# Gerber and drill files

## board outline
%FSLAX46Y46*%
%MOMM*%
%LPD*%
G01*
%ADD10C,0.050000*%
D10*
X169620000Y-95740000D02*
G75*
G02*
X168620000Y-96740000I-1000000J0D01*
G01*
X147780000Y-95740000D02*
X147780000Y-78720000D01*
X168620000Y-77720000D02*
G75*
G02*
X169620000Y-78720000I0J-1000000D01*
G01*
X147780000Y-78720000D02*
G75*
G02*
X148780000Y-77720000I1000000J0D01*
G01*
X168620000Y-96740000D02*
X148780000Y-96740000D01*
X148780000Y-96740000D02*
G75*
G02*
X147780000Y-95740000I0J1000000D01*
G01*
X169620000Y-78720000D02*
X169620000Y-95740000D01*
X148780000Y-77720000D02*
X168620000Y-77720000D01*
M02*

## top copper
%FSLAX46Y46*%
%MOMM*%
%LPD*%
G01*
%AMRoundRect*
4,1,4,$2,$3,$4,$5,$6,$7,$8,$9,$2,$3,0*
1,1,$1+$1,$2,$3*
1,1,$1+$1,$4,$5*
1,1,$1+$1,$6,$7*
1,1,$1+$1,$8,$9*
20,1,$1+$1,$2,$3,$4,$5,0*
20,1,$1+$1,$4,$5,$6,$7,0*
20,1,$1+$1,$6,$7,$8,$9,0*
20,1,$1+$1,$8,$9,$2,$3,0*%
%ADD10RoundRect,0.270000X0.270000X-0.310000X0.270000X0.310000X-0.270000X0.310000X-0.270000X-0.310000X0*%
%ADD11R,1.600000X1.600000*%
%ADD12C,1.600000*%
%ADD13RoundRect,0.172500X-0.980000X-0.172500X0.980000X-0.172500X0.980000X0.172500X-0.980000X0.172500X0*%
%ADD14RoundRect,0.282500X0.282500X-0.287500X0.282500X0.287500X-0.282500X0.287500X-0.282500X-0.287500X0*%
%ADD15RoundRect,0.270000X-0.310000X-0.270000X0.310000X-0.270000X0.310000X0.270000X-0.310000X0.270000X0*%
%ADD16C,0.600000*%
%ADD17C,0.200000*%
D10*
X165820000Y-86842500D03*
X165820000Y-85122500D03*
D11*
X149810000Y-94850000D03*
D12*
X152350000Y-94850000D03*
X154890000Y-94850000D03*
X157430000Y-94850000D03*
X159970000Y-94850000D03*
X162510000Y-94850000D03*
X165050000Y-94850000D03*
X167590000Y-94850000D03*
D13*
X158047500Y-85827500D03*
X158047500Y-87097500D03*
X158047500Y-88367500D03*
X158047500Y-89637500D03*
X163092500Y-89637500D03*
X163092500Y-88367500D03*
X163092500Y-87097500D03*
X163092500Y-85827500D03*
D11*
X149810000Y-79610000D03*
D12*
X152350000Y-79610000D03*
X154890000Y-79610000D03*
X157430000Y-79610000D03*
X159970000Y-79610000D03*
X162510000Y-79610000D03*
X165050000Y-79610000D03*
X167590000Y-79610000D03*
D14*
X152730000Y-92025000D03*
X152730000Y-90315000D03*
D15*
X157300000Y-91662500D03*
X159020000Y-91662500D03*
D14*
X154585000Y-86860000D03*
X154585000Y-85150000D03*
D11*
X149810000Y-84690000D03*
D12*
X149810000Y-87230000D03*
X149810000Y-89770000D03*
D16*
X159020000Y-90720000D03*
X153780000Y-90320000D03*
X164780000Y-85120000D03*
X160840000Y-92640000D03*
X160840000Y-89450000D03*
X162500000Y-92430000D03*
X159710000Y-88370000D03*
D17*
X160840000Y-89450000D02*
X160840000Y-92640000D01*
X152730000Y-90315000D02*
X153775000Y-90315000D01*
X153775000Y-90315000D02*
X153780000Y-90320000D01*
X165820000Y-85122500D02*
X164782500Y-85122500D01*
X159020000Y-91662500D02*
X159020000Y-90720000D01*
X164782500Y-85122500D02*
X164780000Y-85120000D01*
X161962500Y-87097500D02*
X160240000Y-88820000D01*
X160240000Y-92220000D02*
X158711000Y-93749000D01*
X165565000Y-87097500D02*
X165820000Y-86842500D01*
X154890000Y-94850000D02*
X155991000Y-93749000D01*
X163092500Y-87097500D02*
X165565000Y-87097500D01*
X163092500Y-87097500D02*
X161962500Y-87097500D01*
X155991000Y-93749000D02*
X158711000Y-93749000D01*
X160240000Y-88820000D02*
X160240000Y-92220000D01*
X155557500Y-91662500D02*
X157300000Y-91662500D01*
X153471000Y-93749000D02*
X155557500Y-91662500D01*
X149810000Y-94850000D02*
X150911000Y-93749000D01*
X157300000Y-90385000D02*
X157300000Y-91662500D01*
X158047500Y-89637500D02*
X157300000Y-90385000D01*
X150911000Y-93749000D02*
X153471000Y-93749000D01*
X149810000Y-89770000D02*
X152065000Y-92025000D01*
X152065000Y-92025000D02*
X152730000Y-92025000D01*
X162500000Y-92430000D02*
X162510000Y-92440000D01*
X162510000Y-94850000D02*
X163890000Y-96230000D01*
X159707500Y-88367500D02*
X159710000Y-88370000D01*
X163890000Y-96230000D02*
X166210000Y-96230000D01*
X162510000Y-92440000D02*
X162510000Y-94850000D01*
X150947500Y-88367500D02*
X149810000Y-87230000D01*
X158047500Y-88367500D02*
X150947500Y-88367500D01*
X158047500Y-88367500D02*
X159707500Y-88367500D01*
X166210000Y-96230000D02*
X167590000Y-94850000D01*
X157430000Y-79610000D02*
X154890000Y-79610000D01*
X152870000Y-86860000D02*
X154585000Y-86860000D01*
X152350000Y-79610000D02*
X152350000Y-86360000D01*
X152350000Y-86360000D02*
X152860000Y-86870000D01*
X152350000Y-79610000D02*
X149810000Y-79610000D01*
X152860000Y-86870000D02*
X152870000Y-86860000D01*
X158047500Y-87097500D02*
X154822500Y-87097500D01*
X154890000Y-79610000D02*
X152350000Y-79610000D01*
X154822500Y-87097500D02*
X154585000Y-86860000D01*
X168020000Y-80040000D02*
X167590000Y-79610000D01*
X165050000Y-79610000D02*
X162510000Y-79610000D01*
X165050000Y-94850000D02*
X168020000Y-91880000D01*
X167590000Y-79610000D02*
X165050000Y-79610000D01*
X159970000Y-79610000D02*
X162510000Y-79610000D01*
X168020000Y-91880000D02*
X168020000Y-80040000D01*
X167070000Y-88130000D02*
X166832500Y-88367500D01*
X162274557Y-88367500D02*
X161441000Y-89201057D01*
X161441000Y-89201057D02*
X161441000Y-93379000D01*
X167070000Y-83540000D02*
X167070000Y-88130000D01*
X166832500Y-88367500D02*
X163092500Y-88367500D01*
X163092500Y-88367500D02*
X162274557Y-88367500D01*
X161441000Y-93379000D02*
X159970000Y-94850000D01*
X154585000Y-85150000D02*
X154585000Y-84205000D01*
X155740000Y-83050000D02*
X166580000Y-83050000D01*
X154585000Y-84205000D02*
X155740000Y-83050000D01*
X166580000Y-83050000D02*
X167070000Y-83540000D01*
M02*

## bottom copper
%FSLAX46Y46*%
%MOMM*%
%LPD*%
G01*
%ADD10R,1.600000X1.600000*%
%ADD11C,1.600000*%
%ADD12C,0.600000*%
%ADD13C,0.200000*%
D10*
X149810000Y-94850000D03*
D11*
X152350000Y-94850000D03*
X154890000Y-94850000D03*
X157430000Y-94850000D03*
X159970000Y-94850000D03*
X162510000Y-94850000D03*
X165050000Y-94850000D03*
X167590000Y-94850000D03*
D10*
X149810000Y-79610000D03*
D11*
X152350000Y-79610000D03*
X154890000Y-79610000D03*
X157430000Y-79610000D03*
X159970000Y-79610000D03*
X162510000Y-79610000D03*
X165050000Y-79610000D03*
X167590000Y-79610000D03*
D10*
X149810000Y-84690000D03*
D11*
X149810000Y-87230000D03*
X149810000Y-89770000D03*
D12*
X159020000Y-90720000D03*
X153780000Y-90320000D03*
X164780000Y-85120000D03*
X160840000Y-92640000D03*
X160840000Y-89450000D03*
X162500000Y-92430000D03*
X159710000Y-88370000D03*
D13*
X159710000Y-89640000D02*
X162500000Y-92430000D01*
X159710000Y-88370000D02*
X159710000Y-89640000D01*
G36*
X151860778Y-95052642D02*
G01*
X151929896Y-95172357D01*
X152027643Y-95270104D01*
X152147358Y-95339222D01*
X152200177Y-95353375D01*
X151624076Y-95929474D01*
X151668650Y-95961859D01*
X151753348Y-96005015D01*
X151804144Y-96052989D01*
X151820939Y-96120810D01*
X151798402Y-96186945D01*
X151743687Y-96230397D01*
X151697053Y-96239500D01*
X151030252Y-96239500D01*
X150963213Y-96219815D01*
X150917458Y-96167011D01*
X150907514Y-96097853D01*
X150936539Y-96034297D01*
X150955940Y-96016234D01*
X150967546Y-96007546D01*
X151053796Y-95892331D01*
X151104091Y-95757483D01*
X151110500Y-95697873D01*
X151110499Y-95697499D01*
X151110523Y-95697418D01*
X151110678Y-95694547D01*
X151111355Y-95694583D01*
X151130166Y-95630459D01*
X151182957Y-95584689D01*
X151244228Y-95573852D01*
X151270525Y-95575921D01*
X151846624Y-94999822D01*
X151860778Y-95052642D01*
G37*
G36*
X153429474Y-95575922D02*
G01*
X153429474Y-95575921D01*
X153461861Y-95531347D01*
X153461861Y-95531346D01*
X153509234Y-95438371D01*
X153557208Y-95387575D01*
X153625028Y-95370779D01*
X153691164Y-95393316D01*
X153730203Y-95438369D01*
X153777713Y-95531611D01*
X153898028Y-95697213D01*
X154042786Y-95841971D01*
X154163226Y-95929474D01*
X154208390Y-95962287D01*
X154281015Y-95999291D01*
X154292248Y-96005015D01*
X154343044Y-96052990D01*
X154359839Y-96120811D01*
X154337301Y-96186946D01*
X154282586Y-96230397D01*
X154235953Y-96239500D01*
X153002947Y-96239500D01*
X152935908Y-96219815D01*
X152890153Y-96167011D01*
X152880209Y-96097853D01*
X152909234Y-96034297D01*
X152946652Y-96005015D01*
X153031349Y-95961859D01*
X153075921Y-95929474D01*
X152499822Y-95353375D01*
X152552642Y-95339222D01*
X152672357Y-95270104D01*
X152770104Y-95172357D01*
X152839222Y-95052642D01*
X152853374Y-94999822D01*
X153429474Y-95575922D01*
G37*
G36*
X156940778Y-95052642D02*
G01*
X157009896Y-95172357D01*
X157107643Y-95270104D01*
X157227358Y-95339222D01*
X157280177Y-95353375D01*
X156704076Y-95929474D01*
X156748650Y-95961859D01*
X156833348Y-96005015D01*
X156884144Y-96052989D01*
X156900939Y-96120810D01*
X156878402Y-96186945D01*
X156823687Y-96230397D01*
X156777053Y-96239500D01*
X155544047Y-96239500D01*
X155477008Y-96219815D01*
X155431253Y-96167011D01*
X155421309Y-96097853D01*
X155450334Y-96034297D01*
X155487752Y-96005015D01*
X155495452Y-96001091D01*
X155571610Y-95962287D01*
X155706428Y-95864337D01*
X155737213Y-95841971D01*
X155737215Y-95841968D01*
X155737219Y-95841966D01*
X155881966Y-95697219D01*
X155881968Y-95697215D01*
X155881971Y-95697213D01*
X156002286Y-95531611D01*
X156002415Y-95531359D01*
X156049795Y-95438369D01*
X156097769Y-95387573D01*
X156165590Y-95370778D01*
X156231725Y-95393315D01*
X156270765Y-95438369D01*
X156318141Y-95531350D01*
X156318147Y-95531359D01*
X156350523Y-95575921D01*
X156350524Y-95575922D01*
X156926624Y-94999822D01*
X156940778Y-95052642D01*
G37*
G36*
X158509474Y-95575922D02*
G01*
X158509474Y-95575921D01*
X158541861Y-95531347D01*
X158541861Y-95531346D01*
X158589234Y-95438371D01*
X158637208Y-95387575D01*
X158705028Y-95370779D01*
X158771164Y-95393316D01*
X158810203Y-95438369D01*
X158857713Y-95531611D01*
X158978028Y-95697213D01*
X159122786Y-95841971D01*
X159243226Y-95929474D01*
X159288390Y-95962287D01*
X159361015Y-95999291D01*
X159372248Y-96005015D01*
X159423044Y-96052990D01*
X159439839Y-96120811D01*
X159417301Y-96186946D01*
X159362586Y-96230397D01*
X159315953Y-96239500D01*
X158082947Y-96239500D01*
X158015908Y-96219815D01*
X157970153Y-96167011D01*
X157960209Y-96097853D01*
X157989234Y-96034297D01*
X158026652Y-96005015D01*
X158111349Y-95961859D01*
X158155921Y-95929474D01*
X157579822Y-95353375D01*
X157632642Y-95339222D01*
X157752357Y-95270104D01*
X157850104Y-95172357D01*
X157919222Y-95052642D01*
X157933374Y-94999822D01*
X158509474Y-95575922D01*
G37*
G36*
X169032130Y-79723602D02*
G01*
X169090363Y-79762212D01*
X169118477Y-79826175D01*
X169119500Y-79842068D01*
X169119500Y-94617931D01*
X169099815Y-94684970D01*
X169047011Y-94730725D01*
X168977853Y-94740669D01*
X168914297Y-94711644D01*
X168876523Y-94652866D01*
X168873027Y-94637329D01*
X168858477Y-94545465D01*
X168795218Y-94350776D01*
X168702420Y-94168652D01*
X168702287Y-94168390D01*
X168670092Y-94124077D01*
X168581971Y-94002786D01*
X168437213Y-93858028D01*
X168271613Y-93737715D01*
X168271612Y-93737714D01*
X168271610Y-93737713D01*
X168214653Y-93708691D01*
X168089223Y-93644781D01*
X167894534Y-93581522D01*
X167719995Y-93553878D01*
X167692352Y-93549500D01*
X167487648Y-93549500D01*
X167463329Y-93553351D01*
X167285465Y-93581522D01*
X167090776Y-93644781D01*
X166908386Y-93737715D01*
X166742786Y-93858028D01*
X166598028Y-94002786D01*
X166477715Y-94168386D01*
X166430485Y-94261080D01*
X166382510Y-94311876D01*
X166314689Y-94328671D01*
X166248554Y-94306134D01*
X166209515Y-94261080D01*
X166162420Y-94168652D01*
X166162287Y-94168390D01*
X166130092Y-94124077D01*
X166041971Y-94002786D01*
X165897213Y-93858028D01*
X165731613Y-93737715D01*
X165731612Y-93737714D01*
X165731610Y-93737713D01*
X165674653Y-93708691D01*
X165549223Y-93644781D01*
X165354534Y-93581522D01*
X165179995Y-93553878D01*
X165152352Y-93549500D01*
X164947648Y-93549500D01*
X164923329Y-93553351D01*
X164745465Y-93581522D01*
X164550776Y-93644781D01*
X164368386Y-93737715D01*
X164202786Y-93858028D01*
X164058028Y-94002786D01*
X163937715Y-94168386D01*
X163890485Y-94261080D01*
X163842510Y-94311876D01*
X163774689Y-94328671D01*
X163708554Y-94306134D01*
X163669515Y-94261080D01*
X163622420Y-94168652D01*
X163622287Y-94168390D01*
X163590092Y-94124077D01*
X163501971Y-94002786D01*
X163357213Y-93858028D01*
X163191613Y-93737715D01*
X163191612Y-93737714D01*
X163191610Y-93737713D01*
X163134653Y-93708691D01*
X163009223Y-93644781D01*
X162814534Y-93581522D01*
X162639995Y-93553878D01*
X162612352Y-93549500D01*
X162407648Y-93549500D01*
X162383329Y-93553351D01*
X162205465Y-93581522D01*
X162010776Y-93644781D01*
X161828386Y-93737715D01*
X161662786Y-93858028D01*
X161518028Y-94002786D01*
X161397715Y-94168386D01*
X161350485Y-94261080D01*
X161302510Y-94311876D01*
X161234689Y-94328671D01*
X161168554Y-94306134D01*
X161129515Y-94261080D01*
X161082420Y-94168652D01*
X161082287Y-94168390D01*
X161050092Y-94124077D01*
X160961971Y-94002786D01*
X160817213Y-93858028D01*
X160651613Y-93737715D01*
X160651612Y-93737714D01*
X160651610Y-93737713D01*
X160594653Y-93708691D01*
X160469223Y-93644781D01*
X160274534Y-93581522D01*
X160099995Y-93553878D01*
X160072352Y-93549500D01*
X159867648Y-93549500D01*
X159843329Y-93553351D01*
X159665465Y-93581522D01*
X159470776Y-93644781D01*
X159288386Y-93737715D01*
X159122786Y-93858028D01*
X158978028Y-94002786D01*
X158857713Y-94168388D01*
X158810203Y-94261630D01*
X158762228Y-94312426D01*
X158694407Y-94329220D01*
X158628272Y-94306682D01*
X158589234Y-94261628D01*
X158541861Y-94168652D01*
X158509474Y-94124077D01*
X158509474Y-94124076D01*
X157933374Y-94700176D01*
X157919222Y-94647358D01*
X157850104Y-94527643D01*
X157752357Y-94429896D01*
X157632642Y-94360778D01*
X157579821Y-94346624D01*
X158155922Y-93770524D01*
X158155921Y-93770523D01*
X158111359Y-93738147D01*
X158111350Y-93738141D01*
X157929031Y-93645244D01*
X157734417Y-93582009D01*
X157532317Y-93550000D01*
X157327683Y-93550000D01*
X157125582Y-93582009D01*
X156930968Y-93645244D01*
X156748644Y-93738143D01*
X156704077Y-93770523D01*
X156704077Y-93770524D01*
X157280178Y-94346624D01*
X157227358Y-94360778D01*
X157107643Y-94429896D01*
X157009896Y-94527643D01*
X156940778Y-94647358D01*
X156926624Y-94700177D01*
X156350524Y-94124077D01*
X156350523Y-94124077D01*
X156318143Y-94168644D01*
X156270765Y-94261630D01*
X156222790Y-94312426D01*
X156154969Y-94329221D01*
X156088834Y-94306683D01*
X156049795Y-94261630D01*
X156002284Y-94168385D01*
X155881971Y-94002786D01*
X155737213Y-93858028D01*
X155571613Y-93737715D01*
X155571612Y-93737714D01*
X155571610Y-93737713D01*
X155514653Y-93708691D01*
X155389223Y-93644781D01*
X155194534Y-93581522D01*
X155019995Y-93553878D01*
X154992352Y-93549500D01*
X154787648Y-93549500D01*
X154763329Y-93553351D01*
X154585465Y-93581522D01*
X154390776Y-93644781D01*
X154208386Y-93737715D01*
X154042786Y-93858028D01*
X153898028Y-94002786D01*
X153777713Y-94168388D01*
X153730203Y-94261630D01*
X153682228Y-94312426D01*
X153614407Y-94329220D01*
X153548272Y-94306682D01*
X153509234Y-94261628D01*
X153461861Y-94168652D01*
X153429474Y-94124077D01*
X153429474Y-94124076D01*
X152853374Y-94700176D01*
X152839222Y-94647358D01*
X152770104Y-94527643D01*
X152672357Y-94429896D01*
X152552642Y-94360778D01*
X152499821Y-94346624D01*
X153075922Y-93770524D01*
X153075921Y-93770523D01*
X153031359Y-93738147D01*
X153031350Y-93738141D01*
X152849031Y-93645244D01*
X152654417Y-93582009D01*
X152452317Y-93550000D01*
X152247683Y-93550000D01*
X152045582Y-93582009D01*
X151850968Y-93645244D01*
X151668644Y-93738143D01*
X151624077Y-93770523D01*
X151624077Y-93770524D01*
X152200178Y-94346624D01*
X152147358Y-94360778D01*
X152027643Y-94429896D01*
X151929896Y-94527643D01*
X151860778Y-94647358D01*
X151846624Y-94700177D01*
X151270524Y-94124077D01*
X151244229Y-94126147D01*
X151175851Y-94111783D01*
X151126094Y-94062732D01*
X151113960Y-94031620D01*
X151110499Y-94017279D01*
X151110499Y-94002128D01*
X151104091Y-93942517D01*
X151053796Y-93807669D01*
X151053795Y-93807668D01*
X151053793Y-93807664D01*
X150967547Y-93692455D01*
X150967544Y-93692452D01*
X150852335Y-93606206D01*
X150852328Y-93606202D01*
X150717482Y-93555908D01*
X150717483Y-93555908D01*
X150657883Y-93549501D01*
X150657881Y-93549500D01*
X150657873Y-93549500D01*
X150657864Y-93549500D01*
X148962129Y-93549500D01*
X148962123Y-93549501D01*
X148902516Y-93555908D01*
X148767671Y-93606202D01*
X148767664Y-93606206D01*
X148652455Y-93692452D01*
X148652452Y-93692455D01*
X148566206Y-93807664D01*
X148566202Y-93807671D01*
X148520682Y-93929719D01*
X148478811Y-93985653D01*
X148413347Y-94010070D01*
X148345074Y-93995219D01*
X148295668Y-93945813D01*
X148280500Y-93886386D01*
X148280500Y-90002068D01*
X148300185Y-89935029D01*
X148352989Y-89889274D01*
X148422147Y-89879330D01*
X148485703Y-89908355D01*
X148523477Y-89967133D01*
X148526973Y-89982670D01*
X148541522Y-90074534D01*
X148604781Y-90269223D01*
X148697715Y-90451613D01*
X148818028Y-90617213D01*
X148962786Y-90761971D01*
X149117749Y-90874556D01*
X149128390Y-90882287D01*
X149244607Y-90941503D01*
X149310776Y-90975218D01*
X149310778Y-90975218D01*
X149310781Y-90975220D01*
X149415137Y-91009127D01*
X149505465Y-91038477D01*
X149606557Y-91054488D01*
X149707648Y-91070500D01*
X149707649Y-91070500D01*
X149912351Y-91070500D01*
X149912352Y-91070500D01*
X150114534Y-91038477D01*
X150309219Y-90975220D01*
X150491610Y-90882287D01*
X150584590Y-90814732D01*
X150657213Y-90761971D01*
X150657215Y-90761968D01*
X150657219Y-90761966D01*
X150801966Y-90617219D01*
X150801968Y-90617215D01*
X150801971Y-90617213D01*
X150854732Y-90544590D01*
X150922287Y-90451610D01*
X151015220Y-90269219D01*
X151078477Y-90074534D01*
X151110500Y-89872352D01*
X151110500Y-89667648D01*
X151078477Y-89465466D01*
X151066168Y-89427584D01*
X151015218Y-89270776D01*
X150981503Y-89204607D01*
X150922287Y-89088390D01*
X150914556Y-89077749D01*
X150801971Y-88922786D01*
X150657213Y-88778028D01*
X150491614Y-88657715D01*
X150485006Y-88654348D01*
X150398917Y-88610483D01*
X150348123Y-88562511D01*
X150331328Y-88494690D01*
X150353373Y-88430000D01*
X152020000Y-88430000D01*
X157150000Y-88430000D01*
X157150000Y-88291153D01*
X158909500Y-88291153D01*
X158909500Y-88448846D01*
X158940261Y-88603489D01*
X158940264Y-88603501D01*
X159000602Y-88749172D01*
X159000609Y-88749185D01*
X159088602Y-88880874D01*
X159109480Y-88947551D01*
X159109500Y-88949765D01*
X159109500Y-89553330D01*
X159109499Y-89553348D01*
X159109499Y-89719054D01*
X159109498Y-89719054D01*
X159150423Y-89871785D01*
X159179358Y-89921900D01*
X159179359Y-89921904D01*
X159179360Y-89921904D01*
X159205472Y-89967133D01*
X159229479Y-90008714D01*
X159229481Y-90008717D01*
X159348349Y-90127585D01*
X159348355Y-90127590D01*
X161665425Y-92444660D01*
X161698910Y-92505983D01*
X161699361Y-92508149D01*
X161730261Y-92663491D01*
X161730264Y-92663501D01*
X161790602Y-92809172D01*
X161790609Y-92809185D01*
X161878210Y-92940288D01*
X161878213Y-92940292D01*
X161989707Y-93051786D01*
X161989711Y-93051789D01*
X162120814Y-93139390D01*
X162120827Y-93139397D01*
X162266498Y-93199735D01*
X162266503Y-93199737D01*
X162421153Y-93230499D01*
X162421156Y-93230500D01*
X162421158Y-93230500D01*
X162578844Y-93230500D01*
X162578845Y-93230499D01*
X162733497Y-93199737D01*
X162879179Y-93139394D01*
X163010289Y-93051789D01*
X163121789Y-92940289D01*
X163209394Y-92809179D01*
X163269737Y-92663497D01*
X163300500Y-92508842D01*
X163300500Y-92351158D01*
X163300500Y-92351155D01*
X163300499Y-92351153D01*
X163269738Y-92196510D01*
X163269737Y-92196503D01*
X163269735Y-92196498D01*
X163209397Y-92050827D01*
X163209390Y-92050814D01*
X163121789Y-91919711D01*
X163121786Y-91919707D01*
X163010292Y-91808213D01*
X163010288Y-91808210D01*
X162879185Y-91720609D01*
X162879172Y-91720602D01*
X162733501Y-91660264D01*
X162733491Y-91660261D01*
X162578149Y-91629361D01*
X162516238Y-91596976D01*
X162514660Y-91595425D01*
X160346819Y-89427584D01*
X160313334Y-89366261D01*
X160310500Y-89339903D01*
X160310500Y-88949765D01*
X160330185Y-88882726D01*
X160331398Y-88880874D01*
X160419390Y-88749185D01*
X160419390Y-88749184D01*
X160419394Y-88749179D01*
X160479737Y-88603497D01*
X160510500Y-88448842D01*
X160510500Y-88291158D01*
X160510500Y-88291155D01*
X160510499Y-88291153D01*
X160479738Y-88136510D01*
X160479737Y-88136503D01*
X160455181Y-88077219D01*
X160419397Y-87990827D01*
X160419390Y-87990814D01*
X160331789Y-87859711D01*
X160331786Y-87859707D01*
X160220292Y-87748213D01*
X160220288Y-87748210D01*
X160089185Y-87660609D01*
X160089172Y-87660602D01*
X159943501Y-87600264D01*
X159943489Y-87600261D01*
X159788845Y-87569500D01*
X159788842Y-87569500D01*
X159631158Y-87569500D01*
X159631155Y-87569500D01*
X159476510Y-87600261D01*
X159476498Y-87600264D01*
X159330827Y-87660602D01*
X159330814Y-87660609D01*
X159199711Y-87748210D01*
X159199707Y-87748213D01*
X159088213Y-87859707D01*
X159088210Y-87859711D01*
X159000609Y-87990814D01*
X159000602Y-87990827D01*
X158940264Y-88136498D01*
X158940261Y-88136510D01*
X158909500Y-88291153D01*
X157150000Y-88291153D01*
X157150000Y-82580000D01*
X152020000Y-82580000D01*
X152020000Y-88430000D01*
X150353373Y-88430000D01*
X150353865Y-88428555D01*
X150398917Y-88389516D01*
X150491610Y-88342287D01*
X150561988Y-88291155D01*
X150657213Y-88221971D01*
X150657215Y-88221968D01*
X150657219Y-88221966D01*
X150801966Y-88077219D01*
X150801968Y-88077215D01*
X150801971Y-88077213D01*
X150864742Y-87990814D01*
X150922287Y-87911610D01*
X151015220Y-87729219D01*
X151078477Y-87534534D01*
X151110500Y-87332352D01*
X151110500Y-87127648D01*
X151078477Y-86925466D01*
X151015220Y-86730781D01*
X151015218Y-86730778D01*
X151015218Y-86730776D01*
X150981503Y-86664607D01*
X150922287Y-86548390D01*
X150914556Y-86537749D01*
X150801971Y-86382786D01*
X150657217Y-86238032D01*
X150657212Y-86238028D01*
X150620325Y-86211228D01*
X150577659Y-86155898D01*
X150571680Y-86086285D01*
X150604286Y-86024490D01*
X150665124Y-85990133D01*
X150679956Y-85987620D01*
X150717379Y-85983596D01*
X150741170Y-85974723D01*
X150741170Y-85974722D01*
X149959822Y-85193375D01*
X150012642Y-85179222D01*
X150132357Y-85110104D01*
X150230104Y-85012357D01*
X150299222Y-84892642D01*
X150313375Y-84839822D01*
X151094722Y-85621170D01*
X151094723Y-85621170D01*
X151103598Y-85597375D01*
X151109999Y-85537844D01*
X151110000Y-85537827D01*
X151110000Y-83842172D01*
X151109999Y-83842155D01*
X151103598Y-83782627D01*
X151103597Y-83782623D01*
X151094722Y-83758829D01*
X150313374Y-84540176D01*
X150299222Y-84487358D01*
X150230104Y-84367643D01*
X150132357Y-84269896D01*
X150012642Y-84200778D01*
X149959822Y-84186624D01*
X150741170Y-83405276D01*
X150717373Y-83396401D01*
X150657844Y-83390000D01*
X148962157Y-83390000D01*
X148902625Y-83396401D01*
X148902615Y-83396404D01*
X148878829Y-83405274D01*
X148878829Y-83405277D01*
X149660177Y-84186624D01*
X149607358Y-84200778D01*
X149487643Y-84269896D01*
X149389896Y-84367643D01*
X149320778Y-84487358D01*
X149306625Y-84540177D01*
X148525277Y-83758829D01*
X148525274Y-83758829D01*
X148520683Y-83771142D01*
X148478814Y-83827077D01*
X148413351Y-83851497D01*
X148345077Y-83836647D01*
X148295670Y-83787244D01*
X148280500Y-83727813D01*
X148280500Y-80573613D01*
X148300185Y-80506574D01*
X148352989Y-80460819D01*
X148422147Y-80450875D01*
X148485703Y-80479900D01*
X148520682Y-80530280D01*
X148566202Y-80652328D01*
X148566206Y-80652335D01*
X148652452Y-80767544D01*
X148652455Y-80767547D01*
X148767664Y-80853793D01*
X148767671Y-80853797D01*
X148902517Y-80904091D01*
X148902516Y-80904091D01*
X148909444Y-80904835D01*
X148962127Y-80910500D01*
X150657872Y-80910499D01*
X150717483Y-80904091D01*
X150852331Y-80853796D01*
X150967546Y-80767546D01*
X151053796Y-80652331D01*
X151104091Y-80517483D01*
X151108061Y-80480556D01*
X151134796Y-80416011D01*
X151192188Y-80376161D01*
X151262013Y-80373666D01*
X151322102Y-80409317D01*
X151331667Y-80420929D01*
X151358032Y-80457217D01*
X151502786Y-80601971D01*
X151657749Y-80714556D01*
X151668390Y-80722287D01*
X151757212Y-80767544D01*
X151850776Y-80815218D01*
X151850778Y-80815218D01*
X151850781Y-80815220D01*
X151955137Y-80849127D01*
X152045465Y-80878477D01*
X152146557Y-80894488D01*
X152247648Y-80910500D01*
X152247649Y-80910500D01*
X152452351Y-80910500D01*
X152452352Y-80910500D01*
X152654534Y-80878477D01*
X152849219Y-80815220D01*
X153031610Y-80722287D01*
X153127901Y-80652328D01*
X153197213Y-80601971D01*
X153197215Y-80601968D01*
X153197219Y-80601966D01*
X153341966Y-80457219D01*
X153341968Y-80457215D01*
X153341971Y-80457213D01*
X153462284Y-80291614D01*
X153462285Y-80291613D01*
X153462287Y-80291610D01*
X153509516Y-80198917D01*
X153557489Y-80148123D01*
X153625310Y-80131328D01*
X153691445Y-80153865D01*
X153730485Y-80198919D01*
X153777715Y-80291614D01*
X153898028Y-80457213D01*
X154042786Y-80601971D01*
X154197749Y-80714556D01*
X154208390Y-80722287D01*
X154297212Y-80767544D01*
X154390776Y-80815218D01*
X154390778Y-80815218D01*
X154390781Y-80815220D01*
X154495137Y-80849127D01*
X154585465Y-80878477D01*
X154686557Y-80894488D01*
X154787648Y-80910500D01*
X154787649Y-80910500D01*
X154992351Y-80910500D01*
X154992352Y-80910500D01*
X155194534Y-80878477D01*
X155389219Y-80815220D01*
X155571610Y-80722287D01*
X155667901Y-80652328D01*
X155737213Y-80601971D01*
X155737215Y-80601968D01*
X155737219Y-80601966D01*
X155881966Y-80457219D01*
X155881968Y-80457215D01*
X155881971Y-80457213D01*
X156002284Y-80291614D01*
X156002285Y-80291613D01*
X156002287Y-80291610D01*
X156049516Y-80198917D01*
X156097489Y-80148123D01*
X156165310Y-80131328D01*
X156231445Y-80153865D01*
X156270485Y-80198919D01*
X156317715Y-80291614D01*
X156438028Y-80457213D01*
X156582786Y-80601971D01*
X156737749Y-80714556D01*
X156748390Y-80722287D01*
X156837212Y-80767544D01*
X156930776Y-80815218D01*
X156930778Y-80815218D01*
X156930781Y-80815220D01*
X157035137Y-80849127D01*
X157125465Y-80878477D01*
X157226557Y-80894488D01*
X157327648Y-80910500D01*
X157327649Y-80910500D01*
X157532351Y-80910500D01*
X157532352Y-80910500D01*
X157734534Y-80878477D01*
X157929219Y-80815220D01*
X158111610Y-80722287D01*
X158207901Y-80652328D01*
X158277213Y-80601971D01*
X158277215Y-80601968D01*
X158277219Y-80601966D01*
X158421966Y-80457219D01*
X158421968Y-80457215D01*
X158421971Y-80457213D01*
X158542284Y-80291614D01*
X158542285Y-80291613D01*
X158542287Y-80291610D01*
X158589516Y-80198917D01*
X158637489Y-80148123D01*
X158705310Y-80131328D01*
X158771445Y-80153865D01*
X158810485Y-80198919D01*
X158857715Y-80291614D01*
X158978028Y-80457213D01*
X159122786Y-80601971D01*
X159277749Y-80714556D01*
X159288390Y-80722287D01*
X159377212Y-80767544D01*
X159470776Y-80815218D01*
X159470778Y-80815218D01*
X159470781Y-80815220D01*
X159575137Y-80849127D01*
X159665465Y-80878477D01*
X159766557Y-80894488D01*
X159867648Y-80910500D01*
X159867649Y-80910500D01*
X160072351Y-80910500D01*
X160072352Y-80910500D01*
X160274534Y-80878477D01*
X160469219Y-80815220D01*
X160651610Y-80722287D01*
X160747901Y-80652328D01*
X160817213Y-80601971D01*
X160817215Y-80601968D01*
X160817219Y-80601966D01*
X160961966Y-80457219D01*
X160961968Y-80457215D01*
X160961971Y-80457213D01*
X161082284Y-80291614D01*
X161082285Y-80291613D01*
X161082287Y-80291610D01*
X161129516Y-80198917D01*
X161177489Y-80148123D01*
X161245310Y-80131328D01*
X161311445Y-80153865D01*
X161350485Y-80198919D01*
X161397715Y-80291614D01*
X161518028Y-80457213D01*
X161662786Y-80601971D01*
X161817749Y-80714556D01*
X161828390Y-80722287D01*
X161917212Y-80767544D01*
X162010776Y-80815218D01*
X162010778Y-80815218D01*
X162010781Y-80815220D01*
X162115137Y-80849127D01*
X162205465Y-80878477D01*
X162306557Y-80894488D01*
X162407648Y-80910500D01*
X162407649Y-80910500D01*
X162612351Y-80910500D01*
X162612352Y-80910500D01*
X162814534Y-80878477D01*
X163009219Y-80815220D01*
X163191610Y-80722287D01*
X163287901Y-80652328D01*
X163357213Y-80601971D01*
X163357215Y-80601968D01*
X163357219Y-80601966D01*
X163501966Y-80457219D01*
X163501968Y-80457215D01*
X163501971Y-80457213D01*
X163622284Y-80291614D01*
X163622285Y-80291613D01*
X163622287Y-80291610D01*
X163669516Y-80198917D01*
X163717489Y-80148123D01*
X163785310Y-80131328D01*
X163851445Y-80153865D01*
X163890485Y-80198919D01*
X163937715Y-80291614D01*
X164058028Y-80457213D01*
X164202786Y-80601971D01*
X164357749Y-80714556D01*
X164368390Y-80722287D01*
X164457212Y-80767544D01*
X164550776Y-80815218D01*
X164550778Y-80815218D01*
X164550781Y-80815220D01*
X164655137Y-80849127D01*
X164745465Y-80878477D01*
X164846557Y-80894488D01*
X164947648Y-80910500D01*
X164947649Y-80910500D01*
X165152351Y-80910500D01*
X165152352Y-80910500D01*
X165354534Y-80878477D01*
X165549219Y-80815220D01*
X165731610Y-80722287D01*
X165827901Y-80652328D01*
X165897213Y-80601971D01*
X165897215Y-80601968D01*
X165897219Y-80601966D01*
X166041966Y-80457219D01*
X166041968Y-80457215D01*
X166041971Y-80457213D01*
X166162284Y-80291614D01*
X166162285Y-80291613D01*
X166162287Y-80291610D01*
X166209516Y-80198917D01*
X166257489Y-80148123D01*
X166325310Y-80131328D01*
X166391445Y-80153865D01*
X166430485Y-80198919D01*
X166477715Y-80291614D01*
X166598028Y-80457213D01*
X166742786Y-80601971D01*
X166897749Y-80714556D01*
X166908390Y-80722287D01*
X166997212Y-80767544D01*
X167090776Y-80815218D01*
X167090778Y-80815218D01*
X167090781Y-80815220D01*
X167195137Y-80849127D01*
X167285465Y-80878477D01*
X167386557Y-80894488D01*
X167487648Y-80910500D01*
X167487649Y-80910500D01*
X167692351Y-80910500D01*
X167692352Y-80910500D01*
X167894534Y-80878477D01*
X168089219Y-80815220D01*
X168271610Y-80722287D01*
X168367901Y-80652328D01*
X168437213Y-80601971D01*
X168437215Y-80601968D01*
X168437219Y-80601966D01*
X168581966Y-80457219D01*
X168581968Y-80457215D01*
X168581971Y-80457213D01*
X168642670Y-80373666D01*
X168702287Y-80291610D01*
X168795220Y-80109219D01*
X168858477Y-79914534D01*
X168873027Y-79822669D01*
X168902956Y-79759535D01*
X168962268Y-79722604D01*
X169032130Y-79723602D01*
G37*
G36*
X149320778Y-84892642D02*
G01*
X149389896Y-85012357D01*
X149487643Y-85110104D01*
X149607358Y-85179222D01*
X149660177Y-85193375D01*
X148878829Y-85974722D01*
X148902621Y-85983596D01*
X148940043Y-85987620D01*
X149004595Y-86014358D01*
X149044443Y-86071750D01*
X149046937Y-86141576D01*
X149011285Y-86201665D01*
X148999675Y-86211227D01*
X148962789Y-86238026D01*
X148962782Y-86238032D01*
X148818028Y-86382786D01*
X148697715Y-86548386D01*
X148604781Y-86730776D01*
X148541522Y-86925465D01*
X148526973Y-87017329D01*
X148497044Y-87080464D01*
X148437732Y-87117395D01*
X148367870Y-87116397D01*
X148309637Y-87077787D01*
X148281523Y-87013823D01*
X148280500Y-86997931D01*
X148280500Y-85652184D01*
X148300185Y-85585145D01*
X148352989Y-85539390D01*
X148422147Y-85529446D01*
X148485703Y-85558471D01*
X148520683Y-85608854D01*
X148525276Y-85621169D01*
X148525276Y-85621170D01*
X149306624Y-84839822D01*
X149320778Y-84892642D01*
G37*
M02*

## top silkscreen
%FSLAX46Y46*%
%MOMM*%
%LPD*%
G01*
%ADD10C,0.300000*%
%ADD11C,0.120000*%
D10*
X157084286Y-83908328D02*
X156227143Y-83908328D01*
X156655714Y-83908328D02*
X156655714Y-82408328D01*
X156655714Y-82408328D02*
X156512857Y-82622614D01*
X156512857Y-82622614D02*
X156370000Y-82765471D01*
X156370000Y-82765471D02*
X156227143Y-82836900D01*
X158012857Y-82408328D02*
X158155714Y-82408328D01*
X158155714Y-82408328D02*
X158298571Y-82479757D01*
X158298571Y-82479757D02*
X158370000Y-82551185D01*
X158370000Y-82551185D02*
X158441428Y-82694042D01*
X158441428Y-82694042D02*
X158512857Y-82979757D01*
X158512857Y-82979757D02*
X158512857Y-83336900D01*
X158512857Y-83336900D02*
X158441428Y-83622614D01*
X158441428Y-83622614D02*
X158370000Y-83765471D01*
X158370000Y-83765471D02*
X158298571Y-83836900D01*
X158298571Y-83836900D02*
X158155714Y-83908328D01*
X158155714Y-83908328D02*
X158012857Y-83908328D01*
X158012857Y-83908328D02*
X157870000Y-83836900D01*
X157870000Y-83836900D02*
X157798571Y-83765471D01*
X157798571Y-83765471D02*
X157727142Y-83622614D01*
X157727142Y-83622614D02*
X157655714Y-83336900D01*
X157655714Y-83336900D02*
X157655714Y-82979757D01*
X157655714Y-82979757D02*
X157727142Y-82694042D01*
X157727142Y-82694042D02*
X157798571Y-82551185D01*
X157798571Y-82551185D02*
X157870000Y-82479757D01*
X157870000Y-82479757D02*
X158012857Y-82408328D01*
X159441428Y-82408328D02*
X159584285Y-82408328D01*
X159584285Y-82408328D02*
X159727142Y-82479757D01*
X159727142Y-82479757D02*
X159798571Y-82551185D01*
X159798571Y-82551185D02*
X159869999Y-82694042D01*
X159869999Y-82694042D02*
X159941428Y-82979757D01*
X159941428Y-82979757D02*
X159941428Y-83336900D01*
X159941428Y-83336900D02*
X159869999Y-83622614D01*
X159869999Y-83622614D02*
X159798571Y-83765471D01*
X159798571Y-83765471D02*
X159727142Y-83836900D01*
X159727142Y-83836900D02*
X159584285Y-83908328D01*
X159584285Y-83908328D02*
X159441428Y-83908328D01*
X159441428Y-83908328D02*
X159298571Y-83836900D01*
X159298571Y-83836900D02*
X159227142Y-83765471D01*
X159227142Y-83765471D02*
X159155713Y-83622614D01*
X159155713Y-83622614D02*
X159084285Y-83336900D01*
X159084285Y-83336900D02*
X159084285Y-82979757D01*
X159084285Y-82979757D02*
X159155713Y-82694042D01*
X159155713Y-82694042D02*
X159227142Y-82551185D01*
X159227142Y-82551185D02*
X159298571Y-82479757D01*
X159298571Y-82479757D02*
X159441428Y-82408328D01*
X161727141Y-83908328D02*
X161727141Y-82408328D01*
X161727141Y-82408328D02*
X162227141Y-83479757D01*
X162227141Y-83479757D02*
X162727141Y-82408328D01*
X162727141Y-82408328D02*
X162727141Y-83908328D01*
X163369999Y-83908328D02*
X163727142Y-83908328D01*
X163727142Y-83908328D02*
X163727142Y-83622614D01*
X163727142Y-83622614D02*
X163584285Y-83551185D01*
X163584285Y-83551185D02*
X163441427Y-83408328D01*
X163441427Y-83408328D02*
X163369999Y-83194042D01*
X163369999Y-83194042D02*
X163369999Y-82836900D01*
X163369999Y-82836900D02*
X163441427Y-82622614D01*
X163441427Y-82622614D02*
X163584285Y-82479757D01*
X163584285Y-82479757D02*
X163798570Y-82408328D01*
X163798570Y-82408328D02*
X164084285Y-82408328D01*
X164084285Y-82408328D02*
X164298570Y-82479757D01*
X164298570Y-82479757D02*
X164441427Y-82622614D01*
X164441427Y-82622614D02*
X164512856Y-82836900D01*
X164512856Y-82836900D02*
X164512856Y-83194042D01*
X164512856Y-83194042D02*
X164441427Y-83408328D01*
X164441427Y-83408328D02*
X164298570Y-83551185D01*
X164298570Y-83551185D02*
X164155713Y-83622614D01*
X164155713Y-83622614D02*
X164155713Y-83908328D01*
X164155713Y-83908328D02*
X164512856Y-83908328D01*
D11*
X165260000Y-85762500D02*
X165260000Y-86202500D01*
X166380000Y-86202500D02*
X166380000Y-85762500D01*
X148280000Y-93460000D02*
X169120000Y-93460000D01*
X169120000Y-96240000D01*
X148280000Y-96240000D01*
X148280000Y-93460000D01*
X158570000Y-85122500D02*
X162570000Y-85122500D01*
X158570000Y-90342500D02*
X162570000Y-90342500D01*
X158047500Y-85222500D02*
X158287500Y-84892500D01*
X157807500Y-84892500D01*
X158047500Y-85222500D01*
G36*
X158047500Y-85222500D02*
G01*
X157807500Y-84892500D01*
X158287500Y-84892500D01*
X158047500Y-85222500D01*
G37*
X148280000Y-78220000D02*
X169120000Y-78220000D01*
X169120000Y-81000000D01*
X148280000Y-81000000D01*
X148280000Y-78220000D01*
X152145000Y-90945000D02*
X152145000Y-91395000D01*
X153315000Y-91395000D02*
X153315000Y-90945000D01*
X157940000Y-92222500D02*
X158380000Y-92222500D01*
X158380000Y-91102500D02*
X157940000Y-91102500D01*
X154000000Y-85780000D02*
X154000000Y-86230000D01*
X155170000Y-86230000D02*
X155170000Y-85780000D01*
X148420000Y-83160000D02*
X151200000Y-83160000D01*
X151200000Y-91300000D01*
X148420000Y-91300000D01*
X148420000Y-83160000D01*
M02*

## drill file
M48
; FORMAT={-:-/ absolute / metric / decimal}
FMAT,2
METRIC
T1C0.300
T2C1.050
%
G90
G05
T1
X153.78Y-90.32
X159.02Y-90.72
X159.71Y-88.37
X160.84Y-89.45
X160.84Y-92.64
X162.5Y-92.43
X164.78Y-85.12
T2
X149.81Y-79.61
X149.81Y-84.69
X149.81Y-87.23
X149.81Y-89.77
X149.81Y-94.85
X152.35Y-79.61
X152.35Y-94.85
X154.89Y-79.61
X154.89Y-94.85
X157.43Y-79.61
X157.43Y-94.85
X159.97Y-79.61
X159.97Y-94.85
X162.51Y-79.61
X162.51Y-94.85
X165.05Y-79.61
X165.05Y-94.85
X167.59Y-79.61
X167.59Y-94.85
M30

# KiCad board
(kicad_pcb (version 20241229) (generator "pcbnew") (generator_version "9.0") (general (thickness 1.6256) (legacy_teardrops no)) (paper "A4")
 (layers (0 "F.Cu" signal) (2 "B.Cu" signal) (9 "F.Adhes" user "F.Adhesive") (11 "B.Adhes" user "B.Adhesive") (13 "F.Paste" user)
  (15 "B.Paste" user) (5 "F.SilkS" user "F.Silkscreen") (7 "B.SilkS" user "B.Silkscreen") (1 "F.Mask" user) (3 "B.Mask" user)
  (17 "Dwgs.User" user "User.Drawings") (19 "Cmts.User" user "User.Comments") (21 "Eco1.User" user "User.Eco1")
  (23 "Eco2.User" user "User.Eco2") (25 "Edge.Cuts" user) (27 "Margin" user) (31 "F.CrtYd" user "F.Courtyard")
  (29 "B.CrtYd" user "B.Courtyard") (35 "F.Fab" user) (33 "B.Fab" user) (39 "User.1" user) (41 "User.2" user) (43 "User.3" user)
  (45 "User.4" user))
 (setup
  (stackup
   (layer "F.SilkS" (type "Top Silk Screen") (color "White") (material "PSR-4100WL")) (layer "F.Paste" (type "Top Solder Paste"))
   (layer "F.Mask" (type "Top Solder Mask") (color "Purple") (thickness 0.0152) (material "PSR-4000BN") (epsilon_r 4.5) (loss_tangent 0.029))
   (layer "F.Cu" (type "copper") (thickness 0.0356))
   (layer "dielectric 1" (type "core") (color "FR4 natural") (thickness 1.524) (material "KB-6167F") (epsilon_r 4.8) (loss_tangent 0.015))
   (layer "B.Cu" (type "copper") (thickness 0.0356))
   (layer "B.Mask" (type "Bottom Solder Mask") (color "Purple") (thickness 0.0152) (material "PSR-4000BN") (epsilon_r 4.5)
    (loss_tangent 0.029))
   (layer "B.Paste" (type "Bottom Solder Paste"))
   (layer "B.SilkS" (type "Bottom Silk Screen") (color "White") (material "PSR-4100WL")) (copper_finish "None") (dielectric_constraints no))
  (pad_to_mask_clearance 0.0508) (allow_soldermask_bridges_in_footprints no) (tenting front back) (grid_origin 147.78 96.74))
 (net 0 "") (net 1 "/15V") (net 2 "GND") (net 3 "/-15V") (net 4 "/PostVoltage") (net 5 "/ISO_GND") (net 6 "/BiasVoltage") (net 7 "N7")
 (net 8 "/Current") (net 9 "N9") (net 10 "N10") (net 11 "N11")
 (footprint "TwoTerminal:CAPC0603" (layer "F.Cu") (at 165.82 85.9825 90)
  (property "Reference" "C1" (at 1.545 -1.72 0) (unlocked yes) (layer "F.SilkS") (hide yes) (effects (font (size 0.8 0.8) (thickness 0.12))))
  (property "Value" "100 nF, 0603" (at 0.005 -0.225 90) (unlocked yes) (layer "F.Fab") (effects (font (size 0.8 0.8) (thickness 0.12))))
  (fp_line (start 0.22 -0.56) (end -0.22 -0.56) (stroke (width 0.12) (type default)) (layer "F.SilkS"))
  (fp_line (start -0.22 0.56) (end 0.22 0.56) (stroke (width 0.12) (type default)) (layer "F.SilkS"))
  (pad "1" smd roundrect (at -0.86 0 90) (size 1.16 1.08) (layers "F.Cu" "F.Mask" "F.Paste") (roundrect_rratio 0.25) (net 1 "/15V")
   (thermal_bridge_angle 45))
  (pad "2" smd roundrect (at 0.86 0 90) (size 1.16 1.08) (layers "F.Cu" "F.Mask" "F.Paste") (roundrect_rratio 0.25) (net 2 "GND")
   (thermal_bridge_angle 45)))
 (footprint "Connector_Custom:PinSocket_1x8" (layer "F.Cu") (at 158.7 94.85 90)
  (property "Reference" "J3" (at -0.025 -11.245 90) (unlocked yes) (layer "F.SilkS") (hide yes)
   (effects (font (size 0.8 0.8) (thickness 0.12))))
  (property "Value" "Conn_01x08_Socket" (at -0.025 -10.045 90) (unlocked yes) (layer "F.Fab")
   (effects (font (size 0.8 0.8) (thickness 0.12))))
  (fp_rect (start -1.39 -10.42) (end 1.39 10.42) (stroke (width 0.12) (type default)) (fill no) (layer "F.SilkS"))
  (pad "1" thru_hole rect (at 0 -8.89 90) (size 1.6 1.6) (drill 1.05) (layers "*.Cu" "*.Mask") (remove_unused_layers no) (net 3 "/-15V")
   (thermal_bridge_angle 45))
  (pad "2" thru_hole circle (at 0 -6.35 90) (size 1.6 1.6) (drill 1.05) (layers "*.Cu" "*.Mask") (remove_unused_layers no) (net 2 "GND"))
  (pad "3" thru_hole circle (at 0 -3.81 90) (size 1.6 1.6) (drill 1.05) (layers "*.Cu" "*.Mask") (remove_unused_layers no) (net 1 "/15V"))
  (pad "4" thru_hole circle (at 0 -1.27 90) (size 1.6 1.6) (drill 1.05) (layers "*.Cu" "*.Mask") (remove_unused_layers no) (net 2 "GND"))
  (pad "5" thru_hole circle (at 0 1.27 90) (size 1.6 1.6) (drill 1.05) (layers "*.Cu" "*.Mask") (remove_unused_layers no)
   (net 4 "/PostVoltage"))
  (pad "6" thru_hole circle (at 0 3.81 90) (size 1.6 1.6) (drill 1.05) (layers "*.Cu" "*.Mask") (remove_unused_layers no) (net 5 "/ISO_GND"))
  (pad "7" thru_hole circle (at 0 6.35 90) (size 1.6 1.6) (drill 1.05) (layers "*.Cu" "*.Mask") (remove_unused_layers no)
   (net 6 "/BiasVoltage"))
  (pad "8" thru_hole circle (at 0 8.89 90) (size 1.6 1.6) (drill 1.05) (layers "*.Cu" "*.Mask") (remove_unused_layers no) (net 5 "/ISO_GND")))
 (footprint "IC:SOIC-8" (layer "F.Cu") (at 160.57 87.7325)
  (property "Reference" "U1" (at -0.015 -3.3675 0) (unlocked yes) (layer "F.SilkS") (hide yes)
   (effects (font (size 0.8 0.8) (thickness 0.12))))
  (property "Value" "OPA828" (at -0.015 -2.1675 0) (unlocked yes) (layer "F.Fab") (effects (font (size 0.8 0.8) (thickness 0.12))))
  (fp_line (start -2 -2.61) (end 2 -2.61) (stroke (width 0.12) (type default)) (layer "F.SilkS"))
  (fp_line (start -2 2.61) (end 2 2.61) (stroke (width 0.12) (type default)) (layer "F.SilkS"))
  (fp_poly (pts (xy -2.5225 -2.51) (xy -2.2825 -2.84) (xy -2.7625 -2.84)) (stroke (width 0.12) (type solid)) (fill yes) (layer "F.SilkS"))
  (pad "1" smd roundrect (at -2.5225 -1.905) (size 2.305 0.69) (layers "F.Cu" "F.Mask" "F.Paste") (roundrect_rratio 0.25) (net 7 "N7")
   (thermal_bridge_angle 45))
  (pad "2" smd roundrect (at -2.5225 -0.635) (size 2.305 0.69) (layers "F.Cu" "F.Mask" "F.Paste") (roundrect_rratio 0.25) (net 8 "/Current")
   (thermal_bridge_angle 45))
  (pad "3" smd roundrect (at -2.5225 0.635) (size 2.305 0.69) (layers "F.Cu" "F.Mask" "F.Paste") (roundrect_rratio 0.25) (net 5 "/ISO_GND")
   (thermal_bridge_angle 45))
  (pad "4" smd roundrect (at -2.5225 1.905) (size 2.305 0.69) (layers "F.Cu" "F.Mask" "F.Paste") (roundrect_rratio 0.25) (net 3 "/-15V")
   (thermal_bridge_angle 45))
  (pad "5" smd roundrect (at 2.5225 1.905) (size 2.305 0.69) (layers "F.Cu" "F.Mask" "F.Paste") (roundrect_rratio 0.25) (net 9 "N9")
   (thermal_bridge_angle 45))
  (pad "6" smd roundrect (at 2.5225 0.635) (size 2.305 0.69) (layers "F.Cu" "F.Mask" "F.Paste") (roundrect_rratio 0.25)
   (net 4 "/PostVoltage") (thermal_bridge_angle 45))
  (pad "7" smd roundrect (at 2.5225 -0.635) (size 2.305 0.69) (layers "F.Cu" "F.Mask" "F.Paste") (roundrect_rratio 0.25) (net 1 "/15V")
   (thermal_bridge_angle 45))
  (pad "8" smd roundrect (at 2.5225 -1.905) (size 2.305 0.69) (layers "F.Cu" "F.Mask" "F.Paste") (roundrect_rratio 0.25) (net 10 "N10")
   (thermal_bridge_angle 45)))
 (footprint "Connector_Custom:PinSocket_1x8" (layer "F.Cu") (at 158.7 79.61 90)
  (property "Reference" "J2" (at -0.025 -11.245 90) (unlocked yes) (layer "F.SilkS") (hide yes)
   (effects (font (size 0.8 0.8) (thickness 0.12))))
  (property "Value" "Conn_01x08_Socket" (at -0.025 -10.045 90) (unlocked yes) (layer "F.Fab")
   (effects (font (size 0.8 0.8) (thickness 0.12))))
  (fp_rect (start -1.39 -10.42) (end 1.39 10.42) (stroke (width 0.12) (type default)) (fill no) (layer "F.SilkS"))
  (pad "1" thru_hole rect (at 0 -8.89 90) (size 1.6 1.6) (drill 1.05) (layers "*.Cu" "*.Mask") (remove_unused_layers no) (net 8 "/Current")
   (thermal_bridge_angle 45))
  (pad "2" thru_hole circle (at 0 -6.35 90) (size 1.6 1.6) (drill 1.05) (layers "*.Cu" "*.Mask") (remove_unused_layers no)
   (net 8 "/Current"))
  (pad "3" thru_hole circle (at 0 -3.81 90) (size 1.6 1.6) (drill 1.05) (layers "*.Cu" "*.Mask") (remove_unused_layers no)
   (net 8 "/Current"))
  (pad "4" thru_hole circle (at 0 -1.27 90) (size 1.6 1.6) (drill 1.05) (layers "*.Cu" "*.Mask") (remove_unused_layers no)
   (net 8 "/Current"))
  (pad "5" thru_hole circle (at 0 1.27 90) (size 1.6 1.6) (drill 1.05) (layers "*.Cu" "*.Mask") (remove_unused_layers no)
   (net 6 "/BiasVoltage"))
  (pad "6" thru_hole circle (at 0 3.81 90) (size 1.6 1.6) (drill 1.05) (layers "*.Cu" "*.Mask") (remove_unused_layers no)
   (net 6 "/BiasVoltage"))
  (pad "7" thru_hole circle (at 0 6.35 90) (size 1.6 1.6) (drill 1.05) (layers "*.Cu" "*.Mask") (remove_unused_layers no)
   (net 6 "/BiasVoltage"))
  (pad "8" thru_hole circle (at 0 8.89 90) (size 1.6 1.6) (drill 1.05) (layers "*.Cu" "*.Mask") (remove_unused_layers no)
   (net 6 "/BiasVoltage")))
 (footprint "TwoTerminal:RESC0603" (layer "F.Cu") (at 152.73 91.17 90)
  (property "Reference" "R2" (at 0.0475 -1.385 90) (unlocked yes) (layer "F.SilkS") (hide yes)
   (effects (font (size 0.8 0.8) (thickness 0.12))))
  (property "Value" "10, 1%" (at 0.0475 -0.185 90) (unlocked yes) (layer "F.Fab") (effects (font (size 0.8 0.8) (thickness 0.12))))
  (fp_line (start 0.225 -0.585) (end -0.225 -0.585) (stroke (width 0.12) (type default)) (layer "F.SilkS"))
  (fp_line (start -0.225 0.585) (end 0.225 0.585) (stroke (width 0.12) (type default)) (layer "F.SilkS"))
  (pad "1" smd roundrect (at -0.855 0 90) (size 1.14 1.13) (layers "F.Cu" "F.Mask" "F.Paste") (roundrect_rratio 0.25) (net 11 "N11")
   (thermal_bridge_angle 45))
  (pad "2" smd roundrect (at 0.855 0 90) (size 1.14 1.13) (layers "F.Cu" "F.Mask" "F.Paste") (roundrect_rratio 0.25) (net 2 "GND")
   (thermal_bridge_angle 45)))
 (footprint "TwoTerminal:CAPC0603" (layer "F.Cu") (at 158.16 91.6625)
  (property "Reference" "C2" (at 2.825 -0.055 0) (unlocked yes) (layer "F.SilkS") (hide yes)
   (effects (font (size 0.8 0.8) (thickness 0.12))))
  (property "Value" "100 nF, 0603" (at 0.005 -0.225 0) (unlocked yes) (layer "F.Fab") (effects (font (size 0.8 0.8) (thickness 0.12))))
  (fp_line (start -0.22 0.56) (end 0.22 0.56) (stroke (width 0.12) (type default)) (layer "F.SilkS"))
  (fp_line (start 0.22 -0.56) (end -0.22 -0.56) (stroke (width 0.12) (type default)) (layer "F.SilkS"))
  (pad "1" smd roundrect (at -0.86 0) (size 1.16 1.08) (layers "F.Cu" "F.Mask" "F.Paste") (roundrect_rratio 0.25) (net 3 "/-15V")
   (thermal_bridge_angle 45))
  (pad "2" smd roundrect (at 0.86 0) (size 1.16 1.08) (layers "F.Cu" "F.Mask" "F.Paste") (roundrect_rratio 0.25) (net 2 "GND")
   (thermal_bridge_angle 45)))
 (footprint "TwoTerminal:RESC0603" (layer "F.Cu") (at 154.585 86.005 90)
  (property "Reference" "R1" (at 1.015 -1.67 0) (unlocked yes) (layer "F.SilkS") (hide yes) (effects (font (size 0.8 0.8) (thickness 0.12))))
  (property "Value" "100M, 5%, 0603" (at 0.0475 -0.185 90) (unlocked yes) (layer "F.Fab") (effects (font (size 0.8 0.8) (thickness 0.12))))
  (fp_line (start 0.225 -0.585) (end -0.225 -0.585) (stroke (width 0.12) (type default)) (layer "F.SilkS"))
  (fp_line (start -0.225 0.585) (end 0.225 0.585) (stroke (width 0.12) (type default)) (layer "F.SilkS"))
  (pad "1" smd roundrect (at -0.855 0 90) (size 1.14 1.13) (layers "F.Cu" "F.Mask" "F.Paste") (roundrect_rratio 0.25) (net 8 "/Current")
   (thermal_bridge_angle 45))
  (pad "2" smd roundrect (at 0.855 0 90) (size 1.14 1.13) (layers "F.Cu" "F.Mask" "F.Paste") (roundrect_rratio 0.25) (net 4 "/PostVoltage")
   (thermal_bridge_angle 45)))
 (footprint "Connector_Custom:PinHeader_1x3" (layer "F.Cu") (at 149.81 87.23)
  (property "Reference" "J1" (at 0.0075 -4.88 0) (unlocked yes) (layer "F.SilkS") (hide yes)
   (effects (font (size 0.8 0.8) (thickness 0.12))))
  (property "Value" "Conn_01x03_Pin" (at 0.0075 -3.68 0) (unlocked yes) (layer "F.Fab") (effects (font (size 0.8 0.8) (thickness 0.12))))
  (fp_rect (start -1.39 -4.07) (end 1.39 4.07) (stroke (width 0.12) (type default)) (fill no) (layer "F.SilkS"))
  (pad "1" thru_hole rect (at 0 -2.54) (size 1.6 1.6) (drill 1.05) (layers "*.Cu" "*.Mask") (remove_unused_layers no) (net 2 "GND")
   (thermal_bridge_angle 45))
  (pad "2" thru_hole circle (at 0 0) (size 1.6 1.6) (drill 1.05) (layers "*.Cu" "*.Mask") (remove_unused_layers no) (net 5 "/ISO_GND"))
  (pad "3" thru_hole circle (at 0 2.54) (size 1.6 1.6) (drill 1.05) (layers "*.Cu" "*.Mask") (remove_unused_layers no) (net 11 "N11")))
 (gr_arc (start 169.62 95.74) (mid 169.327107 96.447107) (end 168.62 96.74) (stroke (width 0.05) (type default)) (layer "Edge.Cuts"))
 (gr_line (start 147.78 95.74) (end 147.78 78.72) (stroke (width 0.05) (type default)) (layer "Edge.Cuts"))
 (gr_arc (start 168.62 77.72) (mid 169.327107 78.012893) (end 169.62 78.72) (stroke (width 0.05) (type default)) (layer "Edge.Cuts"))
 (gr_arc (start 147.78 78.72) (mid 148.072893 78.012893) (end 148.78 77.72) (stroke (width 0.05) (type default)) (layer "Edge.Cuts"))
 (gr_line (start 168.62 96.74) (end 148.78 96.74) (stroke (width 0.05) (type default)) (layer "Edge.Cuts"))
 (gr_arc (start 148.78 96.74) (mid 148.072893 96.447107) (end 147.78 95.74) (stroke (width 0.05) (type default)) (layer "Edge.Cuts"))
 (gr_line (start 169.62 78.72) (end 169.62 95.74) (stroke (width 0.05) (type default)) (layer "Edge.Cuts"))
 (gr_line (start 148.78 77.72) (end 168.62 77.72) (stroke (width 0.05) (type default)) (layer "Edge.Cuts"))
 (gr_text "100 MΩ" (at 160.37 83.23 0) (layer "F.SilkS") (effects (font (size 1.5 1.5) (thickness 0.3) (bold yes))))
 (segment (start 160.84 89.45) (end 160.84 92.64) (width 0.2) (layer "F.Cu") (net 2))
 (segment (start 152.73 90.315) (end 153.775 90.315) (width 0.2) (layer "F.Cu") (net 2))
 (segment (start 153.775 90.315) (end 153.78 90.32) (width 0.2) (layer "F.Cu") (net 2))
 (segment (start 165.82 85.1225) (end 164.7825 85.1225) (width 0.2) (layer "F.Cu") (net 2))
 (segment (start 159.02 91.6625) (end 159.02 90.72) (width 0.2) (layer "F.Cu") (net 2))
 (segment (start 164.7825 85.1225) (end 164.78 85.12) (width 0.2) (layer "F.Cu") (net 2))
 (via (at 159.02 90.72) (size 0.6) (drill 0.3) (layers "F.Cu" "B.Cu") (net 2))
 (via (at 153.78 90.32) (size 0.6) (drill 0.3) (layers "F.Cu" "B.Cu") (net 2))
 (via (at 164.78 85.12) (size 0.6) (drill 0.3) (layers "F.Cu" "B.Cu") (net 2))
 (via (at 160.84 92.64) (size 0.6) (drill 0.3) (layers "F.Cu" "B.Cu") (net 2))
 (via (at 160.84 89.45) (size 0.6) (drill 0.3) (layers "F.Cu" "B.Cu") (free yes) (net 2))
 (segment (start 161.9625 87.0975) (end 160.24 88.82) (width 0.2) (layer "F.Cu") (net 1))
 (segment (start 160.24 92.22) (end 158.711 93.749) (width 0.2) (layer "F.Cu") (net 1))
 (segment (start 165.565 87.0975) (end 165.82 86.8425) (width 0.2) (layer "F.Cu") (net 1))
 (segment (start 154.89 94.85) (end 155.991 93.749) (width 0.2) (layer "F.Cu") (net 1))
 (segment (start 163.0925 87.0975) (end 165.565 87.0975) (width 0.2) (layer "F.Cu") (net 1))
 (segment (start 163.0925 87.0975) (end 161.9625 87.0975) (width 0.2) (layer "F.Cu") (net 1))
 (segment (start 155.991 93.749) (end 158.711 93.749) (width 0.2) (layer "F.Cu") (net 1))
 (segment (start 160.24 88.82) (end 160.24 92.22) (width 0.2) (layer "F.Cu") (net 1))
 (segment (start 155.5575 91.6625) (end 157.3 91.6625) (width 0.2) (layer "F.Cu") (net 3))
 (segment (start 153.471 93.749) (end 155.5575 91.6625) (width 0.2) (layer "F.Cu") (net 3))
 (segment (start 149.81 94.85) (end 150.911 93.749) (width 0.2) (layer "F.Cu") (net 3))
 (segment (start 157.3 90.385) (end 157.3 91.6625) (width 0.2) (layer "F.Cu") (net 3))
 (segment (start 158.0475 89.6375) (end 157.3 90.385) (width 0.2) (layer "F.Cu") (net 3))
 (segment (start 150.911 93.749) (end 153.471 93.749) (width 0.2) (layer "F.Cu") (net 3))
 (segment (start 149.81 89.77) (end 152.065 92.025) (width 0.2) (layer "F.Cu") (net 11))
 (segment (start 152.065 92.025) (end 152.73 92.025) (width 0.2) (layer "F.Cu") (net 11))
 (segment (start 162.5 92.43) (end 162.51 92.44) (width 0.2) (layer "F.Cu") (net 5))
 (segment (start 162.51 94.85) (end 163.89 96.23) (width 0.2) (layer "F.Cu") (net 5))
 (segment (start 159.7075 88.3675) (end 159.71 88.37) (width 0.2) (layer "F.Cu") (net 5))
 (segment (start 163.89 96.23) (end 166.21 96.23) (width 0.2) (layer "F.Cu") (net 5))
 (segment (start 162.51 92.44) (end 162.51 94.85) (width 0.2) (layer "F.Cu") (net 5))
 (segment (start 150.9475 88.3675) (end 149.81 87.23) (width 0.2) (layer "F.Cu") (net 5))
 (segment (start 158.0475 88.3675) (end 150.9475 88.3675) (width 0.2) (layer "F.Cu") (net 5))
 (segment (start 158.0475 88.3675) (end 159.7075 88.3675) (width 0.2) (layer "F.Cu") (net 5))
 (segment (start 166.21 96.23) (end 167.59 94.85) (width 0.2) (layer "F.Cu") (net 5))
 (via (at 162.5 92.43) (size 0.6) (drill 0.3) (layers "F.Cu" "B.Cu") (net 5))
 (via (at 159.71 88.37) (size 0.6) (drill 0.3) (layers "F.Cu" "B.Cu") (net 5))
 (segment (start 159.71 89.64) (end 162.5 92.43) (width 0.2) (layer "B.Cu") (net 5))
 (segment (start 159.71 88.37) (end 159.71 89.64) (width 0.2) (layer "B.Cu") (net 5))
 (segment (start 157.43 79.61) (end 154.89 79.61) (width 0.2) (layer "F.Cu") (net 8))
 (segment (start 152.87 86.86) (end 154.585 86.86) (width 0.2) (layer "F.Cu") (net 8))
 (segment (start 152.35 79.61) (end 152.35 86.36) (width 0.2) (layer "F.Cu") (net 8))
 (segment (start 152.35 86.36) (end 152.86 86.87) (width 0.2) (layer "F.Cu") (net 8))
 (segment (start 152.35 79.61) (end 149.81 79.61) (width 0.2) (layer "F.Cu") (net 8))
 (segment (start 152.86 86.87) (end 152.87 86.86) (width 0.2) (layer "F.Cu") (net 8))
 (segment (start 158.0475 87.0975) (end 154.8225 87.0975) (width 0.2) (layer "F.Cu") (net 8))
 (segment (start 154.89 79.61) (end 152.35 79.61) (width 0.2) (layer "F.Cu") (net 8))
 (segment (start 154.8225 87.0975) (end 154.585 86.86) (width 0.2) (layer "F.Cu") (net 8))
 (segment (start 168.02 80.04) (end 167.59 79.61) (width 0.2) (layer "F.Cu") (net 6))
 (segment (start 165.05 79.61) (end 162.51 79.61) (width 0.2) (layer "F.Cu") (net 6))
 (segment (start 165.05 94.85) (end 168.02 91.88) (width 0.2) (layer "F.Cu") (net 6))
 (segment (start 167.59 79.61) (end 165.05 79.61) (width 0.2) (layer "F.Cu") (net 6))
 (segment (start 159.97 79.61) (end 162.51 79.61) (width 0.2) (layer "F.Cu") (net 6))
 (segment (start 168.02 91.88) (end 168.02 80.04) (width 0.2) (layer "F.Cu") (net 6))
 (segment (start 167.07 88.13) (end 166.8325 88.3675) (width 0.2) (layer "F.Cu") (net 4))
 (segment (start 162.274557 88.3675) (end 161.441 89.201057) (width 0.2) (layer "F.Cu") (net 4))
 (segment (start 161.441 89.201057) (end 161.441 93.379) (width 0.2) (layer "F.Cu") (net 4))
 (segment (start 167.07 83.54) (end 167.07 88.13) (width 0.2) (layer "F.Cu") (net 4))
 (segment (start 166.8325 88.3675) (end 163.0925 88.3675) (width 0.2) (layer "F.Cu") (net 4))
 (segment (start 163.0925 88.3675) (end 162.274557 88.3675) (width 0.2) (layer "F.Cu") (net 4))
 (segment (start 161.441 93.379) (end 159.97 94.85) (width 0.2) (layer "F.Cu") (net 4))
 (segment (start 154.585 85.15) (end 154.585 84.205) (width 0.2) (layer "F.Cu") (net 4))
 (segment (start 155.74 83.05) (end 166.58 83.05) (width 0.2) (layer "F.Cu") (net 4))
 (segment (start 154.585 84.205) (end 155.74 83.05) (width 0.2) (layer "F.Cu") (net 4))
 (segment (start 166.58 83.05) (end 167.07 83.54) (width 0.2) (layer "F.Cu") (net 4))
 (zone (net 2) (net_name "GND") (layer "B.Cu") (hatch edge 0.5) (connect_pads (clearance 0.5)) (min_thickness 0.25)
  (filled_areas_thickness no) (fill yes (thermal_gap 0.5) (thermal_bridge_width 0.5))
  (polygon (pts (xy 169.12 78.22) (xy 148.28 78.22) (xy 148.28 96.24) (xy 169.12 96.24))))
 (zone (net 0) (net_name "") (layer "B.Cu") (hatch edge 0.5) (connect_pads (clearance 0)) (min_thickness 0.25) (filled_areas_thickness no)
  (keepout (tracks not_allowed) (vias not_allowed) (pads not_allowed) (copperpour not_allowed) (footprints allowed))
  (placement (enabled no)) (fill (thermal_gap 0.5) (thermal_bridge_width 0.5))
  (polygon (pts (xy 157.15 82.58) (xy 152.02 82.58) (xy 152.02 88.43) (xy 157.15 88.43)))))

